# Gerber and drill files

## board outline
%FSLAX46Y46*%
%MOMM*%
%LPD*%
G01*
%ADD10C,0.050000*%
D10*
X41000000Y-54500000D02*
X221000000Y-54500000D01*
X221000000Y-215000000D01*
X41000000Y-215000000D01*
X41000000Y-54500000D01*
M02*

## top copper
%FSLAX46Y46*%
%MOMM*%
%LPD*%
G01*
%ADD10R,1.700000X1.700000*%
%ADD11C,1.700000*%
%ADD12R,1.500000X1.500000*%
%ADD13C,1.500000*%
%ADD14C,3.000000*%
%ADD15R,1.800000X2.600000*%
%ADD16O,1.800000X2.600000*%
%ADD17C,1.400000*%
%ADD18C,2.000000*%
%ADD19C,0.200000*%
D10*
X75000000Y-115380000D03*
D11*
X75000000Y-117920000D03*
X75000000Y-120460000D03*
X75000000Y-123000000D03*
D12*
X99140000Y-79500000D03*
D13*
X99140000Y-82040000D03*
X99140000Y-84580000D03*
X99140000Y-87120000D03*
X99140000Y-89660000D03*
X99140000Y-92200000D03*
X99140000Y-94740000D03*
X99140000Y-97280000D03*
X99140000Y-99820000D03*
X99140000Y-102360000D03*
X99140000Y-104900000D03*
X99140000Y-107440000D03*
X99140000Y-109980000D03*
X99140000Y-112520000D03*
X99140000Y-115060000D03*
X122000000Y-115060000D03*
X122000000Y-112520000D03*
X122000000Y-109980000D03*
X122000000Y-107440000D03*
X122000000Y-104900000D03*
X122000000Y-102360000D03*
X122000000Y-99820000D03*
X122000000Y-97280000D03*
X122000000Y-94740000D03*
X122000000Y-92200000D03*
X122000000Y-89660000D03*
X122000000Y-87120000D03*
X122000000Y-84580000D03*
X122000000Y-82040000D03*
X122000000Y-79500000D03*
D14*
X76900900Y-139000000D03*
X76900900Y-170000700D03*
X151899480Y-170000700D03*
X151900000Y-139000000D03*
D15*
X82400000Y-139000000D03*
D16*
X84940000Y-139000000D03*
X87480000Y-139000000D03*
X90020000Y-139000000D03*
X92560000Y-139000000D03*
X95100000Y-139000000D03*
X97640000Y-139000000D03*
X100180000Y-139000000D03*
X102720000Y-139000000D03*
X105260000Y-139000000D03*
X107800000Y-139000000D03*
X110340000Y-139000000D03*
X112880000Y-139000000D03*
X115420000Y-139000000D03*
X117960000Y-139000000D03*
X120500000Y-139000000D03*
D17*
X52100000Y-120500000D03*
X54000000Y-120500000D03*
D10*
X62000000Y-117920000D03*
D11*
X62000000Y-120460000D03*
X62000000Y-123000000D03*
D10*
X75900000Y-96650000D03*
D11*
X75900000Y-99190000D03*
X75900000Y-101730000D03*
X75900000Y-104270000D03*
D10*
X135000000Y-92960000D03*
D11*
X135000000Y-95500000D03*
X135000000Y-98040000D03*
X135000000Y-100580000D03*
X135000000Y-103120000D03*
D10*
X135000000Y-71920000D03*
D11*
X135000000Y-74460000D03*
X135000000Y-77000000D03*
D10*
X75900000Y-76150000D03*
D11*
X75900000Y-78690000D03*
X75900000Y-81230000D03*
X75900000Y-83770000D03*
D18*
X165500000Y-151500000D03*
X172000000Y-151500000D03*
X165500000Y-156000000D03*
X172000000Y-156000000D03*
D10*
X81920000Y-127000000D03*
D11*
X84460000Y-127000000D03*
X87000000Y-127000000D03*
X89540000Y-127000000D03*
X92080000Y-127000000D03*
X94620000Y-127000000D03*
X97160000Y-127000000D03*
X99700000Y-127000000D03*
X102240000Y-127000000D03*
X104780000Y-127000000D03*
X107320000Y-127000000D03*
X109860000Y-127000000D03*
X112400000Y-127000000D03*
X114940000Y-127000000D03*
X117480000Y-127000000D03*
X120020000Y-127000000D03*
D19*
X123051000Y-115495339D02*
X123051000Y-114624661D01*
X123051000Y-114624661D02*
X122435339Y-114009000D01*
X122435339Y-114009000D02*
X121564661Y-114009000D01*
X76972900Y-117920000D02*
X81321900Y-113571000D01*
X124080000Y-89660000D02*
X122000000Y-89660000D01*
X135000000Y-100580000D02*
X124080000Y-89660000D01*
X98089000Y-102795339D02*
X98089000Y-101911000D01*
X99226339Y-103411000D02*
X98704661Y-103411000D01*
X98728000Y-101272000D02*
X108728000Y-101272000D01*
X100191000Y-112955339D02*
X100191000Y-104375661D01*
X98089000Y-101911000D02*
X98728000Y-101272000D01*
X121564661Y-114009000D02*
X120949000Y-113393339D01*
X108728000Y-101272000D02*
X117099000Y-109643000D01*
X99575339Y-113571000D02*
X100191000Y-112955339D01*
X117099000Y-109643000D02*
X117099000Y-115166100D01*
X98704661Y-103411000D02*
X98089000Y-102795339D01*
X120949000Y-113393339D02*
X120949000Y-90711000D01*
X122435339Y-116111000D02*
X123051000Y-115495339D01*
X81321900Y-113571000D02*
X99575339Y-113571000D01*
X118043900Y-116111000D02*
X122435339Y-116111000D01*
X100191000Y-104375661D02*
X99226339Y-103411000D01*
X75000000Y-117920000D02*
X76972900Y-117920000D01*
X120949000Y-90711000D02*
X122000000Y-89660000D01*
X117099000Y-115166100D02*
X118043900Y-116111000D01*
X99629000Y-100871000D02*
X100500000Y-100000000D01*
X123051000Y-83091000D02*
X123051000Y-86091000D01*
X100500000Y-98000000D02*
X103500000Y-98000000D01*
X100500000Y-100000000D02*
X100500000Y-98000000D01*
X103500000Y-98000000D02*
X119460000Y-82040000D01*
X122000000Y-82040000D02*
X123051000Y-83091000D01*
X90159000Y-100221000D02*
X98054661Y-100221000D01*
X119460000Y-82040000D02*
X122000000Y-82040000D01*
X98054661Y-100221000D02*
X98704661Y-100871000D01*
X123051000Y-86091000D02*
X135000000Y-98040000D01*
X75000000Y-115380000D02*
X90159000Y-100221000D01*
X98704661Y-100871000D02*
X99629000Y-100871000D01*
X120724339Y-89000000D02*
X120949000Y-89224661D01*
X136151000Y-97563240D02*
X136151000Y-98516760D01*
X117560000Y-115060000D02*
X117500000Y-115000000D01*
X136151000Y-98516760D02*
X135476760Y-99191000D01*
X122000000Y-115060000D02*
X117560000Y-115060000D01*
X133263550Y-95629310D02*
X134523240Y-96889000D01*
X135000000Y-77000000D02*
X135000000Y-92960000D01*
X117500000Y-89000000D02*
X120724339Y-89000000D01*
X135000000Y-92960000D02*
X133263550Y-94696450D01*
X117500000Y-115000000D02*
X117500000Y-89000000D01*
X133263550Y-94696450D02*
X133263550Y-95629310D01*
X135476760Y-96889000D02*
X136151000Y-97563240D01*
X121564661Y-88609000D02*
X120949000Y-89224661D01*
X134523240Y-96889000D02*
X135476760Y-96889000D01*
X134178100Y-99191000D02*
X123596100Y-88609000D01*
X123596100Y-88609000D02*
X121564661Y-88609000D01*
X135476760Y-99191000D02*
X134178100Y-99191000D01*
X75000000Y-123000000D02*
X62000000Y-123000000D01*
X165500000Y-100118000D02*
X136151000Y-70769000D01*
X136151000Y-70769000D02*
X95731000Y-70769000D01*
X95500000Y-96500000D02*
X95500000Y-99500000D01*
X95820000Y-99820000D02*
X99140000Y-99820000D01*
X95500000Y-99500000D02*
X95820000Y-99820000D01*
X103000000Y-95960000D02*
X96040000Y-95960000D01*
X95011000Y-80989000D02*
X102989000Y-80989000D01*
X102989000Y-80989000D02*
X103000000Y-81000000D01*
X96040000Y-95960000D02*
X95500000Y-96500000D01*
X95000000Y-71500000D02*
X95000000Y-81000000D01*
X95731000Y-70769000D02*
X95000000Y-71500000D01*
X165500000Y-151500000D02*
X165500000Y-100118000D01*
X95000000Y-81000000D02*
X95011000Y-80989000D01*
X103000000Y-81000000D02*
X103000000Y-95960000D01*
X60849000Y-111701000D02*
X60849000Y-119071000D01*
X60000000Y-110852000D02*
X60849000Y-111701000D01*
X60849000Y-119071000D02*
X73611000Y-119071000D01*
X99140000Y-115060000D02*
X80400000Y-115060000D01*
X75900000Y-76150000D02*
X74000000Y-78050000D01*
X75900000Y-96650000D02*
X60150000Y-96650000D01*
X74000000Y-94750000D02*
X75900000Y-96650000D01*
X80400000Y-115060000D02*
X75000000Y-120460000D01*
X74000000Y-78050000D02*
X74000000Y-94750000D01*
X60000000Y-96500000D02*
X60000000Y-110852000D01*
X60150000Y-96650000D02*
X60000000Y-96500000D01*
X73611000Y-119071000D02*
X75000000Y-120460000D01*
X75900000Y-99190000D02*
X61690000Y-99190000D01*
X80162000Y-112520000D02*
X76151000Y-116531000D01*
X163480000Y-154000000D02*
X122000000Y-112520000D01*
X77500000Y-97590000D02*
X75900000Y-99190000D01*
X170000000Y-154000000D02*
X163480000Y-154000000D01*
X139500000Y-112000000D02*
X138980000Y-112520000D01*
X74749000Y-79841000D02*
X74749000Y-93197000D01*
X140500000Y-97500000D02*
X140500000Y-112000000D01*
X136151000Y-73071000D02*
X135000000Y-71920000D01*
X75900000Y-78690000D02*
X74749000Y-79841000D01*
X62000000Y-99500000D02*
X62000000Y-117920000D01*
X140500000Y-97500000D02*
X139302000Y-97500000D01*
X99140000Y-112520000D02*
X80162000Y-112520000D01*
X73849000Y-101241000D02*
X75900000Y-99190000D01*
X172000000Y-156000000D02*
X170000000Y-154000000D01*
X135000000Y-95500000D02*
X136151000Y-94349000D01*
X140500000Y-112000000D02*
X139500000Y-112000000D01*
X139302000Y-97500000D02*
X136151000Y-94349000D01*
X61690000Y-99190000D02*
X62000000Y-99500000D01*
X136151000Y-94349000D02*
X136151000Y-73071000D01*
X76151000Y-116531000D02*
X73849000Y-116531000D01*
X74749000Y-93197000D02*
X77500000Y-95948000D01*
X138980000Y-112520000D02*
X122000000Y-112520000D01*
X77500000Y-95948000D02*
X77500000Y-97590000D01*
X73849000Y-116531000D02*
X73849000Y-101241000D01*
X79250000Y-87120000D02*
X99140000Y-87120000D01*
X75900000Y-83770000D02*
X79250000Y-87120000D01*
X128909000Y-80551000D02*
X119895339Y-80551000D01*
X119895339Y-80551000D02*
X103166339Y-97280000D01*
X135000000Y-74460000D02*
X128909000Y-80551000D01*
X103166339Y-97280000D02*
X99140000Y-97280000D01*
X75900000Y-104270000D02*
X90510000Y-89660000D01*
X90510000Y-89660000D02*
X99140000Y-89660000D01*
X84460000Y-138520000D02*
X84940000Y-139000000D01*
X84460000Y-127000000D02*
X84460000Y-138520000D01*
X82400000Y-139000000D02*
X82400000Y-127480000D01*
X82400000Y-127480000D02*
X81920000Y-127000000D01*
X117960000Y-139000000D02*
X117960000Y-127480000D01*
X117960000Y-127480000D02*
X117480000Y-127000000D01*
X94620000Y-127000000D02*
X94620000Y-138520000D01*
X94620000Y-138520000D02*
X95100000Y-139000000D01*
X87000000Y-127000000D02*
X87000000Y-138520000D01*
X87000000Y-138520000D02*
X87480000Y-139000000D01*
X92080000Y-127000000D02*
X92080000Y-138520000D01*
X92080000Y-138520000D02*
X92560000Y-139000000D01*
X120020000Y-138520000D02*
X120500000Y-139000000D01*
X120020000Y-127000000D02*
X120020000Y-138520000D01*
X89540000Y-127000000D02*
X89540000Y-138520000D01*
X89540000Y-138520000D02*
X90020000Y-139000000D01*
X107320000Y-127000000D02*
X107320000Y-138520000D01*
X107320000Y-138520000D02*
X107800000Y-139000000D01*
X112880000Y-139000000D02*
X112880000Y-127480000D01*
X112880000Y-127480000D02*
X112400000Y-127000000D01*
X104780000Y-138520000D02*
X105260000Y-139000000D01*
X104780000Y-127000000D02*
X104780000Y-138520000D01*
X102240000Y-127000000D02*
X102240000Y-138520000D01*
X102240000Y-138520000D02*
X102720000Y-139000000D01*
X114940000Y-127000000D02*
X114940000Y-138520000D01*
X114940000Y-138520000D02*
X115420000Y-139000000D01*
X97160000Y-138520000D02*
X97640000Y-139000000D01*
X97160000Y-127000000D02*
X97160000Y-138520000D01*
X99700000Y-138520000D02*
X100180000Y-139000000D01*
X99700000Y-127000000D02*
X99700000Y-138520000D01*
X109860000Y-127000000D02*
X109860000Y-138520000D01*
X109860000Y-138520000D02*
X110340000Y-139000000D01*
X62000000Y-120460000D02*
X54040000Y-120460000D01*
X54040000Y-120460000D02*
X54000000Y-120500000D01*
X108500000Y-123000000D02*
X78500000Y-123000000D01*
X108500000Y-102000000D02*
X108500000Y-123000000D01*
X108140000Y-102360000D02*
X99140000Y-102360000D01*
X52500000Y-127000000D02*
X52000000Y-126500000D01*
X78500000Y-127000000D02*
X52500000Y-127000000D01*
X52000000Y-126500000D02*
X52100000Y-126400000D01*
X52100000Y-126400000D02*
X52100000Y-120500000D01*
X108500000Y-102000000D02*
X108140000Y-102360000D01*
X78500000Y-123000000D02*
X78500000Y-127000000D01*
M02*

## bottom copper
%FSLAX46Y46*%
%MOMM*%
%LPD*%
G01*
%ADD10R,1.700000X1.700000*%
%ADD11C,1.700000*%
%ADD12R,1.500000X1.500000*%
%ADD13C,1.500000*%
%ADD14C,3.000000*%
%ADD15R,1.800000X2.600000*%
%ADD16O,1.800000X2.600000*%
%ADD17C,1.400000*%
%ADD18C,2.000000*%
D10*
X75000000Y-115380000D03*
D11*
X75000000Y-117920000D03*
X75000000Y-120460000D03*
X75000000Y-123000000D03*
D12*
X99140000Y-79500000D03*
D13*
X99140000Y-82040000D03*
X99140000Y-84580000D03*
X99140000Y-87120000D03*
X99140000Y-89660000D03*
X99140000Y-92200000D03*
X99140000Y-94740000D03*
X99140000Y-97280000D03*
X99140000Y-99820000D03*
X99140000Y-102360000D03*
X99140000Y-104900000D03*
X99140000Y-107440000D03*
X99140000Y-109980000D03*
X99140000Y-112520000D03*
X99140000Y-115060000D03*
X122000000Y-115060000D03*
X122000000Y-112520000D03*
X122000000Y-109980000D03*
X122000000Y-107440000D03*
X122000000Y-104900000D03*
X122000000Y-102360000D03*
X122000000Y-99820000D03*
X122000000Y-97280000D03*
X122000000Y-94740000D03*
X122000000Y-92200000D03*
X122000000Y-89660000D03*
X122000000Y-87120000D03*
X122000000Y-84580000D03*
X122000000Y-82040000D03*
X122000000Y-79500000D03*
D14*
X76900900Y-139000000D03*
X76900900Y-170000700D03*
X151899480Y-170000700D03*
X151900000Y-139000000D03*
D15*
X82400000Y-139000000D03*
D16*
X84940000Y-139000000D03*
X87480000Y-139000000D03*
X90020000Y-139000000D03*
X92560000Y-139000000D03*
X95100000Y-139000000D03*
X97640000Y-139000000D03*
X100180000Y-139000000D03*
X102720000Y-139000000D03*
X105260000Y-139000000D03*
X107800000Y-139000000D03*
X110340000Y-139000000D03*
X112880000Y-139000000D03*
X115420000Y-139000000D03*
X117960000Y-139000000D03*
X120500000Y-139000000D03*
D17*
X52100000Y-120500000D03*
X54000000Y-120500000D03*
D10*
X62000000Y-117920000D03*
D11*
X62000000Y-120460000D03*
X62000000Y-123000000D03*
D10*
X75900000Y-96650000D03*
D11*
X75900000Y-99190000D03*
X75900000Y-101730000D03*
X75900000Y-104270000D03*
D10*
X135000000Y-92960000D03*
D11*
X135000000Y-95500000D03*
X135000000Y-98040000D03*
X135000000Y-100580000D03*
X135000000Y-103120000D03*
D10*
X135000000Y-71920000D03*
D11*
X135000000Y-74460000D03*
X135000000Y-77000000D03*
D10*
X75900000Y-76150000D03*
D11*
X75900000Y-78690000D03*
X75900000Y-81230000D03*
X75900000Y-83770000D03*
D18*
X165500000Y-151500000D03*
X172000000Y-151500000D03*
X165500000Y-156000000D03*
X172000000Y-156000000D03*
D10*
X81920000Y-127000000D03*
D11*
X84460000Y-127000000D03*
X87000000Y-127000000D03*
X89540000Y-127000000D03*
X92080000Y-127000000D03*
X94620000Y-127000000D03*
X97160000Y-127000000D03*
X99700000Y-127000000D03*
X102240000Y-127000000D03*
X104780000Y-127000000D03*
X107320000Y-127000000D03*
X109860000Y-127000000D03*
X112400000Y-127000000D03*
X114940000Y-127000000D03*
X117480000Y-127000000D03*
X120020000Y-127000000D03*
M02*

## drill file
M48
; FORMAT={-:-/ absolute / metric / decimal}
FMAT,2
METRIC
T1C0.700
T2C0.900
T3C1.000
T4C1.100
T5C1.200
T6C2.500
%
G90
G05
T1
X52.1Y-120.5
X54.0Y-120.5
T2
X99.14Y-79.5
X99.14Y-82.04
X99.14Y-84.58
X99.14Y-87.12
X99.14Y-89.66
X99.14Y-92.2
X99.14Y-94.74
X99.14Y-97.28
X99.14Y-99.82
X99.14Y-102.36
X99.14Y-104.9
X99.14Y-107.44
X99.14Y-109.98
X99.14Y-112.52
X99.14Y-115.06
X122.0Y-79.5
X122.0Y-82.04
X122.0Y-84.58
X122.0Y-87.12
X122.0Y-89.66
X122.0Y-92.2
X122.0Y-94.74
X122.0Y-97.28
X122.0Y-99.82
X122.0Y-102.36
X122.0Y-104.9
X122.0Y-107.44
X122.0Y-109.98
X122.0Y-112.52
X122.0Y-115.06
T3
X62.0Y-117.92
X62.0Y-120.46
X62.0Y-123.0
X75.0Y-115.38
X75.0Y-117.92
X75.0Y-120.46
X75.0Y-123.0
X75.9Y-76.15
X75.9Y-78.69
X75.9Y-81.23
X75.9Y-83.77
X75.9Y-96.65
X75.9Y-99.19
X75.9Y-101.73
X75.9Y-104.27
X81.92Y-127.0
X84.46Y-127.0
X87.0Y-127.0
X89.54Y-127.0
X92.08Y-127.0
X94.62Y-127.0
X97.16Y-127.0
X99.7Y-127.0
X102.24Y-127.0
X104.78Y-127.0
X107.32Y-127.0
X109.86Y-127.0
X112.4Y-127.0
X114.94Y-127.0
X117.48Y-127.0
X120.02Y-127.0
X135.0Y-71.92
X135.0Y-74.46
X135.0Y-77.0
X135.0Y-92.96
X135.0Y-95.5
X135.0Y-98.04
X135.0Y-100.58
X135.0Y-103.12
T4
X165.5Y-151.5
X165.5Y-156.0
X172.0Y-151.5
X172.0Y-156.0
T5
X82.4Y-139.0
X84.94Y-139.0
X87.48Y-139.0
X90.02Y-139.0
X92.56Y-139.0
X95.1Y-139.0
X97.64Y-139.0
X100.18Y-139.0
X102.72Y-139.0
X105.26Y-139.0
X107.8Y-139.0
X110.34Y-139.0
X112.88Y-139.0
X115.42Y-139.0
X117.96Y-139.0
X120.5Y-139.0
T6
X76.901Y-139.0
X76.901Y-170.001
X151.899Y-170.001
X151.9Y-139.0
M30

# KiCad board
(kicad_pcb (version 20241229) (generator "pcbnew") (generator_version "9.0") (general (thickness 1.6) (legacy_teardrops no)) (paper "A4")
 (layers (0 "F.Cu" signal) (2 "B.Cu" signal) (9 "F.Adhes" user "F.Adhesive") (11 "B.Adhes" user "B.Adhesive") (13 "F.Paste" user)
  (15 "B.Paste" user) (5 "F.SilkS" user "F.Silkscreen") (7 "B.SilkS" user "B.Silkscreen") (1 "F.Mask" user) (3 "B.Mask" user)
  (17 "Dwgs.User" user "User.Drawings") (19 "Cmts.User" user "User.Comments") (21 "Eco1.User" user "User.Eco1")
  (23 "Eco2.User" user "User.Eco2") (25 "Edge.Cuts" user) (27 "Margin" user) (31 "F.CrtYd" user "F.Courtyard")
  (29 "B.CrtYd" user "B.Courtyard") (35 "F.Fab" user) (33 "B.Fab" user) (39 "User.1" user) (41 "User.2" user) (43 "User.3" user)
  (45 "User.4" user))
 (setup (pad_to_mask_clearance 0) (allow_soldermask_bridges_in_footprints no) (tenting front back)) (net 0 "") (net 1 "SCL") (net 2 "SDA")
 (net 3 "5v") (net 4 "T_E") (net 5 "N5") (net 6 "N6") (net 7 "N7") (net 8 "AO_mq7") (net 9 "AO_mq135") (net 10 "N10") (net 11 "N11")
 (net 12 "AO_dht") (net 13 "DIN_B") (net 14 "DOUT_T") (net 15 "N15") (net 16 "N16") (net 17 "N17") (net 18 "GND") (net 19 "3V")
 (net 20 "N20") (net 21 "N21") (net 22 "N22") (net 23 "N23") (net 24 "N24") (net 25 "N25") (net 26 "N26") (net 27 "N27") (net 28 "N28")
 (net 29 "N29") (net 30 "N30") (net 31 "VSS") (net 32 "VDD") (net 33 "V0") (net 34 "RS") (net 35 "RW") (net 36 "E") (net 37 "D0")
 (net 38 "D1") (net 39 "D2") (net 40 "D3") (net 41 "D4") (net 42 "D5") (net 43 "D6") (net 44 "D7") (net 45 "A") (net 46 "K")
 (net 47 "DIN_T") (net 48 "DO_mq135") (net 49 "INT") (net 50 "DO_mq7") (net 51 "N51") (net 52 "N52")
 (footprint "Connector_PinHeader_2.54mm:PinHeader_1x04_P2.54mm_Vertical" (layer "F.Cu") (at 75 115.38)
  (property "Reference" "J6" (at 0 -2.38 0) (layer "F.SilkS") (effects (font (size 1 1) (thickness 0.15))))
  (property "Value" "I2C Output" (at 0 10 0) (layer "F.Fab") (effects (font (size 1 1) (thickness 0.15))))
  (pad "1" thru_hole rect (at 0 0) (size 1.7 1.7) (drill 1) (layers "*.Cu" "*.Mask") (remove_unused_layers no) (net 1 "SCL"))
  (pad "2" thru_hole circle (at 0 2.54) (size 1.7 1.7) (drill 1) (layers "*.Cu" "*.Mask") (remove_unused_layers no) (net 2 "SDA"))
  (pad "3" thru_hole circle (at 0 5.08) (size 1.7 1.7) (drill 1) (layers "*.Cu" "*.Mask") (remove_unused_layers no) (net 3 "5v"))
  (pad "4" thru_hole circle (at 0 7.62) (size 1.7 1.7) (drill 1) (layers "*.Cu" "*.Mask") (remove_unused_layers no) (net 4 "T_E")))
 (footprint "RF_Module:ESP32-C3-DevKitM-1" (layer "F.Cu") (at 99.14 79.5)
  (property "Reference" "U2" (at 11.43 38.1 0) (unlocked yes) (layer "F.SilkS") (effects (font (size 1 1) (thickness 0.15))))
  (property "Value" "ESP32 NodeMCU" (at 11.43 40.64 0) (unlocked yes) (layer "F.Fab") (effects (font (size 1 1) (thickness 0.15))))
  (pad "1" thru_hole rect (at 0 0) (size 1.5 1.5) (drill 0.9) (layers "*.Cu" "*.Mask") (remove_unused_layers yes) (keep_end_layers yes)
   (zone_layer_connections) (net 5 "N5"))
  (pad "2" thru_hole circle (at 0 2.54) (size 1.5 1.5) (drill 0.9) (layers "*.Cu" "*.Mask") (remove_unused_layers yes) (keep_end_layers yes)
   (zone_layer_connections) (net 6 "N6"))
  (pad "3" thru_hole circle (at 0 5.08) (size 1.5 1.5) (drill 0.9) (layers "*.Cu" "*.Mask") (remove_unused_layers yes) (keep_end_layers yes)
   (zone_layer_connections) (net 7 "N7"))
  (pad "4" thru_hole circle (at 0 7.62) (size 1.5 1.5) (drill 0.9) (layers "*.Cu" "*.Mask") (remove_unused_layers yes) (keep_end_layers yes)
   (zone_layer_connections) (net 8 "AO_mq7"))
  (pad "5" thru_hole circle (at 0 10.16) (size 1.5 1.5) (drill 0.9) (layers "*.Cu" "*.Mask") (remove_unused_layers yes)
   (keep_end_layers yes) (zone_layer_connections) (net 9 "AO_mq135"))
  (pad "6" thru_hole circle (at 0 12.7) (size 1.5 1.5) (drill 0.9) (layers "*.Cu" "*.Mask") (remove_unused_layers yes) (keep_end_layers yes)
   (zone_layer_connections) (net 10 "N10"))
  (pad "7" thru_hole circle (at 0 15.24) (size 1.5 1.5) (drill 0.9) (layers "*.Cu" "*.Mask") (remove_unused_layers yes)
   (keep_end_layers yes) (zone_layer_connections) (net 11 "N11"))
  (pad "8" thru_hole circle (at 0 17.78) (size 1.5 1.5) (drill 0.9) (layers "*.Cu" "*.Mask") (remove_unused_layers yes)
   (keep_end_layers yes) (zone_layer_connections) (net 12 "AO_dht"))
  (pad "9" thru_hole circle (at 0 20.32) (size 1.5 1.5) (drill 0.9) (layers "*.Cu" "*.Mask") (remove_unused_layers yes)
   (keep_end_layers yes) (zone_layer_connections) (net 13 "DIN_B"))
  (pad "10" thru_hole circle (at 0 22.86) (size 1.5 1.5) (drill 0.9) (layers "*.Cu" "*.Mask") (remove_unused_layers yes)
   (keep_end_layers yes) (zone_layer_connections) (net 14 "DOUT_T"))
  (pad "11" thru_hole circle (at 0 25.4) (size 1.5 1.5) (drill 0.9) (layers "*.Cu" "*.Mask") (remove_unused_layers yes)
   (keep_end_layers yes) (zone_layer_connections) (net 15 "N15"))
  (pad "12" thru_hole circle (at 0 27.94) (size 1.5 1.5) (drill 0.9) (layers "*.Cu" "*.Mask") (remove_unused_layers yes)
   (keep_end_layers yes) (zone_layer_connections) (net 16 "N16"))
  (pad "13" thru_hole circle (at 0 30.48) (size 1.5 1.5) (drill 0.9) (layers "*.Cu" "*.Mask") (remove_unused_layers yes)
   (keep_end_layers yes) (zone_layer_connections) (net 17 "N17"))
  (pad "14" thru_hole circle (at 0 33.02) (size 1.5 1.5) (drill 0.9) (layers "*.Cu" "*.Mask") (remove_unused_layers yes)
   (keep_end_layers yes) (zone_layer_connections) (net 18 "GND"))
  (pad "15" thru_hole circle (at 0 35.56) (size 1.5 1.5) (drill 0.9) (layers "*.Cu" "*.Mask") (remove_unused_layers yes)
   (keep_end_layers yes) (zone_layer_connections) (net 3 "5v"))
  (pad "16" thru_hole circle (at 22.86 35.56) (size 1.5 1.5) (drill 0.9) (layers "*.Cu" "*.Mask") (remove_unused_layers yes)
   (keep_end_layers yes) (zone_layer_connections) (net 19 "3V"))
  (pad "17" thru_hole circle (at 22.86 33.02) (size 1.5 1.5) (drill 0.9) (layers "*.Cu" "*.Mask") (remove_unused_layers yes)
   (keep_end_layers yes) (zone_layer_connections) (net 18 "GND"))
  (pad "18" thru_hole circle (at 22.86 30.48) (size 1.5 1.5) (drill 0.9) (layers "*.Cu" "*.Mask") (remove_unused_layers yes)
   (keep_end_layers yes) (zone_layer_connections) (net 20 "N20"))
  (pad "19" thru_hole circle (at 22.86 27.94) (size 1.5 1.5) (drill 0.9) (layers "*.Cu" "*.Mask") (remove_unused_layers yes)
   (keep_end_layers yes) (zone_layer_connections) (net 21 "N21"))
  (pad "20" thru_hole circle (at 22.86 25.4) (size 1.5 1.5) (drill 0.9) (layers "*.Cu" "*.Mask") (remove_unused_layers yes)
   (keep_end_layers yes) (zone_layer_connections) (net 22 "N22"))
  (pad "21" thru_hole circle (at 22.86 22.86) (size 1.5 1.5) (drill 0.9) (layers "*.Cu" "*.Mask") (remove_unused_layers yes)
   (keep_end_layers yes) (zone_layer_connections) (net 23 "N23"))
  (pad "22" thru_hole circle (at 22.86 20.32) (size 1.5 1.5) (drill 0.9) (layers "*.Cu" "*.Mask") (remove_unused_layers yes)
   (keep_end_layers yes) (zone_layer_connections) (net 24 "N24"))
  (pad "23" thru_hole circle (at 22.86 17.78) (size 1.5 1.5) (drill 0.9) (layers "*.Cu" "*.Mask") (remove_unused_layers yes)
   (keep_end_layers yes) (zone_layer_connections) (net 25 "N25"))
  (pad "24" thru_hole circle (at 22.86 15.24) (size 1.5 1.5) (drill 0.9) (layers "*.Cu" "*.Mask") (remove_unused_layers yes)
   (keep_end_layers yes) (zone_layer_connections) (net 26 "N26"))
  (pad "25" thru_hole circle (at 22.86 12.7) (size 1.5 1.5) (drill 0.9) (layers "*.Cu" "*.Mask") (remove_unused_layers yes)
   (keep_end_layers yes) (zone_layer_connections) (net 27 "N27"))
  (pad "26" thru_hole circle (at 22.86 10.16) (size 1.5 1.5) (drill 0.9) (layers "*.Cu" "*.Mask") (remove_unused_layers yes)
   (keep_end_layers yes) (zone_layer_connections) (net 2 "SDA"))
  (pad "27" thru_hole circle (at 22.86 7.62) (size 1.5 1.5) (drill 0.9) (layers "*.Cu" "*.Mask") (remove_unused_layers yes)
   (keep_end_layers yes) (zone_layer_connections) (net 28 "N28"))
  (pad "28" thru_hole circle (at 22.86 5.08) (size 1.5 1.5) (drill 0.9) (layers "*.Cu" "*.Mask") (remove_unused_layers yes)
   (keep_end_layers yes) (zone_layer_connections) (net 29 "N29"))
  (pad "29" thru_hole circle (at 22.86 2.54) (size 1.5 1.5) (drill 0.9) (layers "*.Cu" "*.Mask") (remove_unused_layers yes)
   (keep_end_layers yes) (zone_layer_connections) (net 1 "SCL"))
  (pad "30" thru_hole circle (at 22.86 0) (size 1.5 1.5) (drill 0.9) (layers "*.Cu" "*.Mask") (remove_unused_layers yes)
   (keep_end_layers yes) (zone_layer_connections) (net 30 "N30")))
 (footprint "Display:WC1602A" (layer "F.Cu") (at 82.4 139)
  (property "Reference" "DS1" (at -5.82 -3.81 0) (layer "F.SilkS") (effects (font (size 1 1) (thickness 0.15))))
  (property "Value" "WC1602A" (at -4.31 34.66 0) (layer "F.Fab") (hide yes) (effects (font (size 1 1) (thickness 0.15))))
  (pad "" thru_hole circle (at -5.4991 0) (size 3 3) (drill 2.5) (layers "*.Cu" "*.Mask") (remove_unused_layers no))
  (pad "" thru_hole circle (at -5.4991 31.0007) (size 3 3) (drill 2.5) (layers "*.Cu" "*.Mask") (remove_unused_layers no))
  (pad "" thru_hole circle (at 69.49948 31.0007) (size 3 3) (drill 2.5) (layers "*.Cu" "*.Mask") (remove_unused_layers no))
  (pad "" thru_hole circle (at 69.5 0) (size 3 3) (drill 2.5) (layers "*.Cu" "*.Mask") (remove_unused_layers no))
  (pad "1" thru_hole rect (at 0 0) (size 1.8 2.6) (drill 1.2) (layers "*.Cu" "*.Mask") (remove_unused_layers no) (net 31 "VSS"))
  (pad "2" thru_hole oval (at 2.54 0) (size 1.8 2.6) (drill 1.2) (layers "*.Cu" "*.Mask") (remove_unused_layers no) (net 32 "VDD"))
  (pad "3" thru_hole oval (at 5.08 0) (size 1.8 2.6) (drill 1.2) (layers "*.Cu" "*.Mask") (remove_unused_layers no) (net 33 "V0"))
  (pad "4" thru_hole oval (at 7.62 0) (size 1.8 2.6) (drill 1.2) (layers "*.Cu" "*.Mask") (remove_unused_layers no) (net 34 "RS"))
  (pad "5" thru_hole oval (at 10.16 0) (size 1.8 2.6) (drill 1.2) (layers "*.Cu" "*.Mask") (remove_unused_layers no) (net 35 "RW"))
  (pad "6" thru_hole oval (at 12.7 0) (size 1.8 2.6) (drill 1.2) (layers "*.Cu" "*.Mask") (remove_unused_layers no) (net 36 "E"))
  (pad "7" thru_hole oval (at 15.24 0) (size 1.8 2.6) (drill 1.2) (layers "*.Cu" "*.Mask") (remove_unused_layers no) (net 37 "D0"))
  (pad "8" thru_hole oval (at 17.78 0) (size 1.8 2.6) (drill 1.2) (layers "*.Cu" "*.Mask") (remove_unused_layers no) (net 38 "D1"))
  (pad "9" thru_hole oval (at 20.32 0) (size 1.8 2.6) (drill 1.2) (layers "*.Cu" "*.Mask") (remove_unused_layers no) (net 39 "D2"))
  (pad "10" thru_hole oval (at 22.86 0) (size 1.8 2.6) (drill 1.2) (layers "*.Cu" "*.Mask") (remove_unused_layers no) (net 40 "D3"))
  (pad "11" thru_hole oval (at 25.4 0) (size 1.8 2.6) (drill 1.2) (layers "*.Cu" "*.Mask") (remove_unused_layers no) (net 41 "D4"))
  (pad "12" thru_hole oval (at 27.94 0) (size 1.8 2.6) (drill 1.2) (layers "*.Cu" "*.Mask") (remove_unused_layers no) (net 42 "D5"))
  (pad "13" thru_hole oval (at 30.48 0) (size 1.8 2.6) (drill 1.2) (layers "*.Cu" "*.Mask") (remove_unused_layers no) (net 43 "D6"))
  (pad "14" thru_hole oval (at 33.02 0) (size 1.8 2.6) (drill 1.2) (layers "*.Cu" "*.Mask") (remove_unused_layers no) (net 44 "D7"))
  (pad "15" thru_hole oval (at 35.56 0) (size 1.8 2.6) (drill 1.2) (layers "*.Cu" "*.Mask") (remove_unused_layers no) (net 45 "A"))
  (pad "16" thru_hole oval (at 38.1 0) (size 1.8 2.6) (drill 1.2) (layers "*.Cu" "*.Mask") (remove_unused_layers no) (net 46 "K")))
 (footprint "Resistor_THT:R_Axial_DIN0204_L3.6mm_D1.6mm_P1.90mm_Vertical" (layer "F.Cu") (at 52.1 120.5)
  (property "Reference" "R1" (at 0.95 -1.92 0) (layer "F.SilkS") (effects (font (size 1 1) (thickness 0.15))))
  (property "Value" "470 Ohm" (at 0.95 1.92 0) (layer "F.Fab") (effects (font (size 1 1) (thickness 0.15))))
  (pad "1" thru_hole circle (at 0 0) (size 1.4 1.4) (drill 0.7) (layers "*.Cu" "*.Mask") (remove_unused_layers no) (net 14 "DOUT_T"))
  (pad "2" thru_hole circle (at 1.9 0) (size 1.4 1.4) (drill 0.7) (layers "*.Cu" "*.Mask") (remove_unused_layers no) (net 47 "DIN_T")))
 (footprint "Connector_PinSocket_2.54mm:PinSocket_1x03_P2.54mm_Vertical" (layer "F.Cu") (at 62 117.92)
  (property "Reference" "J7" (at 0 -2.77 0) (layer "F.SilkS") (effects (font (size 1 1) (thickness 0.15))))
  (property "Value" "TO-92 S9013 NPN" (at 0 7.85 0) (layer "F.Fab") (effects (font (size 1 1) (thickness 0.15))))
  (pad "1" thru_hole rect (at 0 0) (size 1.7 1.7) (drill 1) (layers "*.Cu" "*.Mask") (remove_unused_layers no) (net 18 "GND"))
  (pad "2" thru_hole circle (at 0 2.54) (size 1.7 1.7) (drill 1) (layers "*.Cu" "*.Mask") (remove_unused_layers no) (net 47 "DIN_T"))
  (pad "3" thru_hole circle (at 0 5.08) (size 1.7 1.7) (drill 1) (layers "*.Cu" "*.Mask") (remove_unused_layers no) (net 4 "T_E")))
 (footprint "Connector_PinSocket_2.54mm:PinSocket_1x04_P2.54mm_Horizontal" (layer "F.Cu") (at 75.9 96.65)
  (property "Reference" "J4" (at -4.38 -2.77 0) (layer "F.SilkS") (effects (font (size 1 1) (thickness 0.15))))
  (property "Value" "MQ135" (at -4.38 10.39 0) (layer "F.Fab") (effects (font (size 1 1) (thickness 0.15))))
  (pad "1" thru_hole rect (at 0 0) (size 1.7 1.7) (drill 1) (layers "*.Cu" "*.Mask") (remove_unused_layers no) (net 3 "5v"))
  (pad "2" thru_hole circle (at 0 2.54) (size 1.7 1.7) (drill 1) (layers "*.Cu" "*.Mask") (remove_unused_layers no) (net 18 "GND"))
  (pad "3" thru_hole circle (at 0 5.08) (size 1.7 1.7) (drill 1) (layers "*.Cu" "*.Mask") (remove_unused_layers no) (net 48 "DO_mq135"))
  (pad "4" thru_hole circle (at 0 7.62) (size 1.7 1.7) (drill 1) (layers "*.Cu" "*.Mask") (remove_unused_layers no) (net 9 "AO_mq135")))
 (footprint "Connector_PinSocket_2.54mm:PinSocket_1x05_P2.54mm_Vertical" (layer "F.Cu") (at 135 92.96)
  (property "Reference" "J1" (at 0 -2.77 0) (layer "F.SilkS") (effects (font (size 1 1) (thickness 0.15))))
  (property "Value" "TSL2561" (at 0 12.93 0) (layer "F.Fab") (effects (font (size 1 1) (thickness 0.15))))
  (pad "1" thru_hole rect (at 0 0) (size 1.7 1.7) (drill 1) (layers "*.Cu" "*.Mask") (remove_unused_layers no) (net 19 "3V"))
  (pad "2" thru_hole circle (at 0 2.54) (size 1.7 1.7) (drill 1) (layers "*.Cu" "*.Mask") (remove_unused_layers no) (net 18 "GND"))
  (pad "3" thru_hole circle (at 0 5.08) (size 1.7 1.7) (drill 1) (layers "*.Cu" "*.Mask") (remove_unused_layers no) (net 1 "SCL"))
  (pad "4" thru_hole circle (at 0 7.62) (size 1.7 1.7) (drill 1) (layers "*.Cu" "*.Mask") (remove_unused_layers no) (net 2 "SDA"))
  (pad "5" thru_hole circle (at 0 10.16) (size 1.7 1.7) (drill 1) (layers "*.Cu" "*.Mask") (remove_unused_layers no) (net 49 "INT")))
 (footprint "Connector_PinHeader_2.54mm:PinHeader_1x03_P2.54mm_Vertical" (layer "F.Cu") (at 135 71.92)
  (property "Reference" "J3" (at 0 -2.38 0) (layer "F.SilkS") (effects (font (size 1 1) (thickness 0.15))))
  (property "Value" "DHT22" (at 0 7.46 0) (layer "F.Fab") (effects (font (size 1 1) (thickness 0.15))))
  (pad "1" thru_hole rect (at 0 0) (size 1.7 1.7) (drill 1) (layers "*.Cu" "*.Mask") (remove_unused_layers no) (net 18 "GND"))
  (pad "2" thru_hole circle (at 0 2.54) (size 1.7 1.7) (drill 1) (layers "*.Cu" "*.Mask") (remove_unused_layers no) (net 12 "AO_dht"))
  (pad "3" thru_hole circle (at 0 5.08) (size 1.7 1.7) (drill 1) (layers "*.Cu" "*.Mask") (remove_unused_layers no) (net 19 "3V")))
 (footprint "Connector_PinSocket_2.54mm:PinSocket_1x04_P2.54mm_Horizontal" (layer "F.Cu") (at 75.9 76.15)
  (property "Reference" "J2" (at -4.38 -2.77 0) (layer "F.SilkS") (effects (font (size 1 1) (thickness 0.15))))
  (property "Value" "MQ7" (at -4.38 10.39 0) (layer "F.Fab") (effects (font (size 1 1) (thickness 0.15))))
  (pad "1" thru_hole rect (at 0 0) (size 1.7 1.7) (drill 1) (layers "*.Cu" "*.Mask") (remove_unused_layers no) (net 3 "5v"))
  (pad "2" thru_hole circle (at 0 2.54) (size 1.7 1.7) (drill 1) (layers "*.Cu" "*.Mask") (remove_unused_layers no) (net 18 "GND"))
  (pad "3" thru_hole circle (at 0 5.08) (size 1.7 1.7) (drill 1) (layers "*.Cu" "*.Mask") (remove_unused_layers no) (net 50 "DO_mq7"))
  (pad "4" thru_hole circle (at 0 7.62) (size 1.7 1.7) (drill 1) (layers "*.Cu" "*.Mask") (remove_unused_layers no) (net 8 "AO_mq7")))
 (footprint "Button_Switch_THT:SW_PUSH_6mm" (layer "F.Cu") (at 165.5 151.5)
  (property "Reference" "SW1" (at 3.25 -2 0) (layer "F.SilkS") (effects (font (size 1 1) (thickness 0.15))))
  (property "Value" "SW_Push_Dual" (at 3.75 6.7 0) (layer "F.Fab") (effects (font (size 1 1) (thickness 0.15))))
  (pad "1" thru_hole circle (at 0 0 90) (size 2 2) (drill 1.1) (layers "*.Cu" "*.Mask") (remove_unused_layers no) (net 13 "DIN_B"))
  (pad "2" thru_hole circle (at 6.5 0 90) (size 2 2) (drill 1.1) (layers "*.Cu" "*.Mask") (remove_unused_layers no) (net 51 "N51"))
  (pad "3" thru_hole circle (at 0 4.5 90) (size 2 2) (drill 1.1) (layers "*.Cu" "*.Mask") (remove_unused_layers no) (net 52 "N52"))
  (pad "4" thru_hole circle (at 6.5 4.5 90) (size 2 2) (drill 1.1) (layers "*.Cu" "*.Mask") (remove_unused_layers no) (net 18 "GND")))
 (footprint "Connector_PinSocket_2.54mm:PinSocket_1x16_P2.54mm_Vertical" (layer "F.Cu") (at 81.92 127 90)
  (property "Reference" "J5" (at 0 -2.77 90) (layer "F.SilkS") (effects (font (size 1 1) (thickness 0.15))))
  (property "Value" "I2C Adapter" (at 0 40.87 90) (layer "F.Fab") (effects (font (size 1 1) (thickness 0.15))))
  (pad "1" thru_hole rect (at 0 0 90) (size 1.7 1.7) (drill 1) (layers "*.Cu" "*.Mask") (remove_unused_layers no) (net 31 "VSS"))
  (pad "2" thru_hole circle (at 0 2.54 90) (size 1.7 1.7) (drill 1) (layers "*.Cu" "*.Mask") (remove_unused_layers no) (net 32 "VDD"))
  (pad "3" thru_hole circle (at 0 5.08 90) (size 1.7 1.7) (drill 1) (layers "*.Cu" "*.Mask") (remove_unused_layers no) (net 33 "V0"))
  (pad "4" thru_hole circle (at 0 7.62 90) (size 1.7 1.7) (drill 1) (layers "*.Cu" "*.Mask") (remove_unused_layers no) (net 34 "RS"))
  (pad "5" thru_hole circle (at 0 10.16 90) (size 1.7 1.7) (drill 1) (layers "*.Cu" "*.Mask") (remove_unused_layers no) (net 35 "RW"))
  (pad "6" thru_hole circle (at 0 12.7 90) (size 1.7 1.7) (drill 1) (layers "*.Cu" "*.Mask") (remove_unused_layers no) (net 36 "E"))
  (pad "7" thru_hole circle (at 0 15.24 90) (size 1.7 1.7) (drill 1) (layers "*.Cu" "*.Mask") (remove_unused_layers no) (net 37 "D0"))
  (pad "8" thru_hole circle (at 0 17.78 90) (size 1.7 1.7) (drill 1) (layers "*.Cu" "*.Mask") (remove_unused_layers no) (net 38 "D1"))
  (pad "9" thru_hole circle (at 0 20.32 90) (size 1.7 1.7) (drill 1) (layers "*.Cu" "*.Mask") (remove_unused_layers no) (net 39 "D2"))
  (pad "10" thru_hole circle (at 0 22.86 90) (size 1.7 1.7) (drill 1) (layers "*.Cu" "*.Mask") (remove_unused_layers no) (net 40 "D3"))
  (pad "11" thru_hole circle (at 0 25.4 90) (size 1.7 1.7) (drill 1) (layers "*.Cu" "*.Mask") (remove_unused_layers no) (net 41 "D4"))
  (pad "12" thru_hole circle (at 0 27.94 90) (size 1.7 1.7) (drill 1) (layers "*.Cu" "*.Mask") (remove_unused_layers no) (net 42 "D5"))
  (pad "13" thru_hole circle (at 0 30.48 90) (size 1.7 1.7) (drill 1) (layers "*.Cu" "*.Mask") (remove_unused_layers no) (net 43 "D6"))
  (pad "14" thru_hole circle (at 0 33.02 90) (size 1.7 1.7) (drill 1) (layers "*.Cu" "*.Mask") (remove_unused_layers no) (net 44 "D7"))
  (pad "15" thru_hole circle (at 0 35.56 90) (size 1.7 1.7) (drill 1) (layers "*.Cu" "*.Mask") (remove_unused_layers no) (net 45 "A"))
  (pad "16" thru_hole circle (at 0 38.1 90) (size 1.7 1.7) (drill 1) (layers "*.Cu" "*.Mask") (remove_unused_layers no) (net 46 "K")))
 (gr_rect (start 41 54.5) (end 221 215) (stroke (width 0.05) (type default)) (fill no) (layer "Edge.Cuts"))
 (segment (start 123.051 115.495339) (end 123.051 114.624661) (width 0.2) (layer "F.Cu") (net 2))
 (segment (start 123.051 114.624661) (end 122.435339 114.009) (width 0.2) (layer "F.Cu") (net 2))
 (segment (start 122.435339 114.009) (end 121.564661 114.009) (width 0.2) (layer "F.Cu") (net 2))
 (segment (start 76.9729 117.92) (end 81.3219 113.571) (width 0.2) (layer "F.Cu") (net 2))
 (segment (start 124.08 89.66) (end 122 89.66) (width 0.2) (layer "F.Cu") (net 2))
 (segment (start 135 100.58) (end 124.08 89.66) (width 0.2) (layer "F.Cu") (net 2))
 (segment (start 98.089 102.795339) (end 98.089 101.911) (width 0.2) (layer "F.Cu") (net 2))
 (segment (start 99.226339 103.411) (end 98.704661 103.411) (width 0.2) (layer "F.Cu") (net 2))
 (segment (start 98.728 101.272) (end 108.728 101.272) (width 0.2) (layer "F.Cu") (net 2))
 (segment (start 100.191 112.955339) (end 100.191 104.375661) (width 0.2) (layer "F.Cu") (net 2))
 (segment (start 98.089 101.911) (end 98.728 101.272) (width 0.2) (layer "F.Cu") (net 2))
 (segment (start 121.564661 114.009) (end 120.949 113.393339) (width 0.2) (layer "F.Cu") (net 2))
 (segment (start 108.728 101.272) (end 117.099 109.643) (width 0.2) (layer "F.Cu") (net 2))
 (segment (start 99.575339 113.571) (end 100.191 112.955339) (width 0.2) (layer "F.Cu") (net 2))
 (segment (start 117.099 109.643) (end 117.099 115.1661) (width 0.2) (layer "F.Cu") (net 2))
 (segment (start 98.704661 103.411) (end 98.089 102.795339) (width 0.2) (layer "F.Cu") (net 2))
 (segment (start 120.949 113.393339) (end 120.949 90.711) (width 0.2) (layer "F.Cu") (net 2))
 (segment (start 122.435339 116.111) (end 123.051 115.495339) (width 0.2) (layer "F.Cu") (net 2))
 (segment (start 81.3219 113.571) (end 99.575339 113.571) (width 0.2) (layer "F.Cu") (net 2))
 (segment (start 118.0439 116.111) (end 122.435339 116.111) (width 0.2) (layer "F.Cu") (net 2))
 (segment (start 100.191 104.375661) (end 99.226339 103.411) (width 0.2) (layer "F.Cu") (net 2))
 (segment (start 75 117.92) (end 76.9729 117.92) (width 0.2) (layer "F.Cu") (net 2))
 (segment (start 120.949 90.711) (end 122 89.66) (width 0.2) (layer "F.Cu") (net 2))
 (segment (start 117.099 115.1661) (end 118.0439 116.111) (width 0.2) (layer "F.Cu") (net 2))
 (segment (start 99.629 100.871) (end 100.5 100) (width 0.2) (layer "F.Cu") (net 1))
 (segment (start 123.051 83.091) (end 123.051 86.091) (width 0.2) (layer "F.Cu") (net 1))
 (segment (start 100.5 98) (end 103.5 98) (width 0.2) (layer "F.Cu") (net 1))
 (segment (start 100.5 100) (end 100.5 98) (width 0.2) (layer "F.Cu") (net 1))
 (segment (start 103.5 98) (end 119.46 82.04) (width 0.2) (layer "F.Cu") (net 1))
 (segment (start 122 82.04) (end 123.051 83.091) (width 0.2) (layer "F.Cu") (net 1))
 (segment (start 90.159 100.221) (end 98.054661 100.221) (width 0.2) (layer "F.Cu") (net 1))
 (segment (start 119.46 82.04) (end 122 82.04) (width 0.2) (layer "F.Cu") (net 1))
 (segment (start 98.054661 100.221) (end 98.704661 100.871) (width 0.2) (layer "F.Cu") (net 1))
 (segment (start 123.051 86.091) (end 135 98.04) (width 0.2) (layer "F.Cu") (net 1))
 (segment (start 75 115.38) (end 90.159 100.221) (width 0.2) (layer "F.Cu") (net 1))
 (segment (start 98.704661 100.871) (end 99.629 100.871) (width 0.2) (layer "F.Cu") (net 1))
 (segment (start 120.724339 89) (end 120.949 89.224661) (width 0.2) (layer "F.Cu") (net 19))
 (segment (start 136.151 97.56324) (end 136.151 98.51676) (width 0.2) (layer "F.Cu") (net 19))
 (segment (start 117.56 115.06) (end 117.5 115) (width 0.2) (layer "F.Cu") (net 19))
 (segment (start 136.151 98.51676) (end 135.47676 99.191) (width 0.2) (layer "F.Cu") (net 19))
 (segment (start 122 115.06) (end 117.56 115.06) (width 0.2) (layer "F.Cu") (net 19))
 (segment (start 133.26355 95.62931) (end 134.52324 96.889) (width 0.2) (layer "F.Cu") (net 19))
 (segment (start 135 77) (end 135 92.96) (width 0.2) (layer "F.Cu") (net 19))
 (segment (start 117.5 89) (end 120.724339 89) (width 0.2) (layer "F.Cu") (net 19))
 (segment (start 135 92.96) (end 133.26355 94.69645) (width 0.2) (layer "F.Cu") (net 19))
 (segment (start 117.5 115) (end 117.5 89) (width 0.2) (layer "F.Cu") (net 19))
 (segment (start 133.26355 94.69645) (end 133.26355 95.62931) (width 0.2) (layer "F.Cu") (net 19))
 (segment (start 135.47676 96.889) (end 136.151 97.56324) (width 0.2) (layer "F.Cu") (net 19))
 (segment (start 121.564661 88.609) (end 120.949 89.224661) (width 0.2) (layer "F.Cu") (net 19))
 (segment (start 134.52324 96.889) (end 135.47676 96.889) (width 0.2) (layer "F.Cu") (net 19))
 (segment (start 134.1781 99.191) (end 123.5961 88.609) (width 0.2) (layer "F.Cu") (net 19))
 (segment (start 123.5961 88.609) (end 121.564661 88.609) (width 0.2) (layer "F.Cu") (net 19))
 (segment (start 135.47676 99.191) (end 134.1781 99.191) (width 0.2) (layer "F.Cu") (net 19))
 (segment (start 75 123) (end 62 123) (width 0.2) (layer "F.Cu") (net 4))
 (segment (start 165.5 100.118) (end 136.151 70.769) (width 0.2) (layer "F.Cu") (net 13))
 (segment (start 136.151 70.769) (end 95.731 70.769) (width 0.2) (layer "F.Cu") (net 13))
 (segment (start 95.5 96.5) (end 95.5 99.5) (width 0.2) (layer "F.Cu") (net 13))
 (segment (start 95.82 99.82) (end 99.14 99.82) (width 0.2) (layer "F.Cu") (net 13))
 (segment (start 95.5 99.5) (end 95.82 99.82) (width 0.2) (layer "F.Cu") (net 13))
 (segment (start 103 95.96) (end 96.04 95.96) (width 0.2) (layer "F.Cu") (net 13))
 (segment (start 95.011 80.989) (end 102.989 80.989) (width 0.2) (layer "F.Cu") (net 13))
 (segment (start 102.989 80.989) (end 103 81) (width 0.2) (layer "F.Cu") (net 13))
 (segment (start 96.04 95.96) (end 95.5 96.5) (width 0.2) (layer "F.Cu") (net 13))
 (segment (start 95 71.5) (end 95 81) (width 0.2) (layer "F.Cu") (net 13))
 (segment (start 95.731 70.769) (end 95 71.5) (width 0.2) (layer "F.Cu") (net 13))
 (segment (start 165.5 151.5) (end 165.5 100.118) (width 0.2) (layer "F.Cu") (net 13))
 (segment (start 95 81) (end 95.011 80.989) (width 0.2) (layer "F.Cu") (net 13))
 (segment (start 103 81) (end 103 95.96) (width 0.2) (layer "F.Cu") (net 13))
 (segment (start 60.849 111.701) (end 60.849 119.071) (width 0.2) (layer "F.Cu") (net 3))
 (segment (start 60 110.852) (end 60.849 111.701) (width 0.2) (layer "F.Cu") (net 3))
 (segment (start 60.849 119.071) (end 73.611 119.071) (width 0.2) (layer "F.Cu") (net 3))
 (segment (start 99.14 115.06) (end 80.4 115.06) (width 0.2) (layer "F.Cu") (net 3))
 (segment (start 75.9 76.15) (end 74 78.05) (width 0.2) (layer "F.Cu") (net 3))
 (segment (start 75.9 96.65) (end 60.15 96.65) (width 0.2) (layer "F.Cu") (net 3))
 (segment (start 74 94.75) (end 75.9 96.65) (width 0.2) (layer "F.Cu") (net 3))
 (segment (start 80.4 115.06) (end 75 120.46) (width 0.2) (layer "F.Cu") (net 3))
 (segment (start 74 78.05) (end 74 94.75) (width 0.2) (layer "F.Cu") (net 3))
 (segment (start 60 96.5) (end 60 110.852) (width 0.2) (layer "F.Cu") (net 3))
 (segment (start 60.15 96.65) (end 60 96.5) (width 0.2) (layer "F.Cu") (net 3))
 (segment (start 73.611 119.071) (end 75 120.46) (width 0.2) (layer "F.Cu") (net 3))
 (segment (start 75.9 99.19) (end 61.69 99.19) (width 0.2) (layer "F.Cu") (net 18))
 (segment (start 80.162 112.52) (end 76.151 116.531) (width 0.2) (layer "F.Cu") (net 18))
 (segment (start 163.48 154) (end 122 112.52) (width 0.2) (layer "F.Cu") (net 18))
 (segment (start 77.5 97.59) (end 75.9 99.19) (width 0.2) (layer "F.Cu") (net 18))
 (segment (start 170 154) (end 163.48 154) (width 0.2) (layer "F.Cu") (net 18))
 (segment (start 139.5 112) (end 138.98 112.52) (width 0.2) (layer "F.Cu") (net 18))
 (segment (start 74.749 79.841) (end 74.749 93.197) (width 0.2) (layer "F.Cu") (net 18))
 (segment (start 140.5 97.5) (end 140.5 112) (width 0.2) (layer "F.Cu") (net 18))
 (segment (start 136.151 73.071) (end 135 71.92) (width 0.2) (layer "F.Cu") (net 18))
 (segment (start 75.9 78.69) (end 74.749 79.841) (width 0.2) (layer "F.Cu") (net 18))
 (segment (start 62 99.5) (end 62 117.92) (width 0.2) (layer "F.Cu") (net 18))
 (segment (start 140.5 97.5) (end 139.302 97.5) (width 0.2) (layer "F.Cu") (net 18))
 (segment (start 99.14 112.52) (end 80.162 112.52) (width 0.2) (layer "F.Cu") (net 18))
 (segment (start 73.849 101.241) (end 75.9 99.19) (width 0.2) (layer "F.Cu") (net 18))
 (segment (start 172 156) (end 170 154) (width 0.2) (layer "F.Cu") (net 18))
 (segment (start 135 95.5) (end 136.151 94.349) (width 0.2) (layer "F.Cu") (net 18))
 (segment (start 140.5 112) (end 139.5 112) (width 0.2) (layer "F.Cu") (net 18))
 (segment (start 139.302 97.5) (end 136.151 94.349) (width 0.2) (layer "F.Cu") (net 18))
 (segment (start 61.69 99.19) (end 62 99.5) (width 0.2) (layer "F.Cu") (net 18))
 (segment (start 136.151 94.349) (end 136.151 73.071) (width 0.2) (layer "F.Cu") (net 18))
 (segment (start 76.151 116.531) (end 73.849 116.531) (width 0.2) (layer "F.Cu") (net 18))
 (segment (start 74.749 93.197) (end 77.5 95.948) (width 0.2) (layer "F.Cu") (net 18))
 (segment (start 138.98 112.52) (end 122 112.52) (width 0.2) (layer "F.Cu") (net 18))
 (segment (start 77.5 95.948) (end 77.5 97.59) (width 0.2) (layer "F.Cu") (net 18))
 (segment (start 73.849 116.531) (end 73.849 101.241) (width 0.2) (layer "F.Cu") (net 18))
 (segment (start 79.25 87.12) (end 99.14 87.12) (width 0.2) (layer "F.Cu") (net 8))
 (segment (start 75.9 83.77) (end 79.25 87.12) (width 0.2) (layer "F.Cu") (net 8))
 (segment (start 128.909 80.551) (end 119.895339 80.551) (width 0.2) (layer "F.Cu") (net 12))
 (segment (start 119.895339 80.551) (end 103.166339 97.28) (width 0.2) (layer "F.Cu") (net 12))
 (segment (start 135 74.46) (end 128.909 80.551) (width 0.2) (layer "F.Cu") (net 12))
 (segment (start 103.166339 97.28) (end 99.14 97.28) (width 0.2) (layer "F.Cu") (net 12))
 (segment (start 75.9 104.27) (end 90.51 89.66) (width 0.2) (layer "F.Cu") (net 9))
 (segment (start 90.51 89.66) (end 99.14 89.66) (width 0.2) (layer "F.Cu") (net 9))
 (segment (start 84.46 138.52) (end 84.94 139) (width 0.2) (layer "F.Cu") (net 32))
 (segment (start 84.46 127) (end 84.46 138.52) (width 0.2) (layer "F.Cu") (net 32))
 (segment (start 82.4 139) (end 82.4 127.48) (width 0.2) (layer "F.Cu") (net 31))
 (segment (start 82.4 127.48) (end 81.92 127) (width 0.2) (layer "F.Cu") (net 31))
 (segment (start 117.96 139) (end 117.96 127.48) (width 0.2) (layer "F.Cu") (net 45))
 (segment (start 117.96 127.48) (end 117.48 127) (width 0.2) (layer "F.Cu") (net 45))
 (segment (start 94.62 127) (end 94.62 138.52) (width 0.2) (layer "F.Cu") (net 36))
 (segment (start 94.62 138.52) (end 95.1 139) (width 0.2) (layer "F.Cu") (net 36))
 (segment (start 87 127) (end 87 138.52) (width 0.2) (layer "F.Cu") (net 33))
 (segment (start 87 138.52) (end 87.48 139) (width 0.2) (layer "F.Cu") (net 33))
 (segment (start 92.08 127) (end 92.08 138.52) (width 0.2) (layer "F.Cu") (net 35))
 (segment (start 92.08 138.52) (end 92.56 139) (width 0.2) (layer "F.Cu") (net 35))
 (segment (start 120.02 138.52) (end 120.5 139) (width 0.2) (layer "F.Cu") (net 46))
 (segment (start 120.02 127) (end 120.02 138.52) (width 0.2) (layer "F.Cu") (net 46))
 (segment (start 89.54 127) (end 89.54 138.52) (width 0.2) (layer "F.Cu") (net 34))
 (segment (start 89.54 138.52) (end 90.02 139) (width 0.2) (layer "F.Cu") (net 34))
 (segment (start 107.32 127) (end 107.32 138.52) (width 0.2) (layer "F.Cu") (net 41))
 (segment (start 107.32 138.52) (end 107.8 139) (width 0.2) (layer "F.Cu") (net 41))
 (segment (start 112.88 139) (end 112.88 127.48) (width 0.2) (layer "F.Cu") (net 43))
 (segment (start 112.88 127.48) (end 112.4 127) (width 0.2) (layer "F.Cu") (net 43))
 (segment (start 104.78 138.52) (end 105.26 139) (width 0.2) (layer "F.Cu") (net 40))
 (segment (start 104.78 127) (end 104.78 138.52) (width 0.2) (layer "F.Cu") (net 40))
 (segment (start 102.24 127) (end 102.24 138.52) (width 0.2) (layer "F.Cu") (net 39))
 (segment (start 102.24 138.52) (end 102.72 139) (width 0.2) (layer "F.Cu") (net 39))
 (segment (start 114.94 127) (end 114.94 138.52) (width 0.2) (layer "F.Cu") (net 44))
 (segment (start 114.94 138.52) (end 115.42 139) (width 0.2) (layer "F.Cu") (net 44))
 (segment (start 97.16 138.52) (end 97.64 139) (width 0.2) (layer "F.Cu") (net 37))
 (segment (start 97.16 127) (end 97.16 138.52) (width 0.2) (layer "F.Cu") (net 37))
 (segment (start 99.7 138.52) (end 100.18 139) (width 0.2) (layer "F.Cu") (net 38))
 (segment (start 99.7 127) (end 99.7 138.52) (width 0.2) (layer "F.Cu") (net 38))
 (segment (start 109.86 127) (end 109.86 138.52) (width 0.2) (layer "F.Cu") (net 42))
 (segment (start 109.86 138.52) (end 110.34 139) (width 0.2) (layer "F.Cu") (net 42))
 (segment (start 62 120.46) (end 54.04 120.46) (width 0.2) (layer "F.Cu") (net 47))
 (segment (start 54.04 120.46) (end 54 120.5) (width 0.2) (layer "F.Cu") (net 47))
 (segment (start 108.5 123) (end 78.5 123) (width 0.2) (layer "F.Cu") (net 14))
 (segment (start 108.5 102) (end 108.5 123) (width 0.2) (layer "F.Cu") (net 14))
 (segment (start 108.14 102.36) (end 99.14 102.36) (width 0.2) (layer "F.Cu") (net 14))
 (segment (start 52.5 127) (end 52 126.5) (width 0.2) (layer "F.Cu") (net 14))
 (segment (start 78.5 127) (end 52.5 127) (width 0.2) (layer "F.Cu") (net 14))
 (segment (start 52 126.5) (end 52.1 126.4) (width 0.2) (layer "F.Cu") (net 14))
 (segment (start 52.1 126.4) (end 52.1 120.5) (width 0.2) (layer "F.Cu") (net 14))
 (segment (start 108.5 102) (end 108.14 102.36) (width 0.2) (layer "F.Cu") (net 14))
 (segment (start 78.5 123) (end 78.5 127) (width 0.2) (layer "F.Cu") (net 14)))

